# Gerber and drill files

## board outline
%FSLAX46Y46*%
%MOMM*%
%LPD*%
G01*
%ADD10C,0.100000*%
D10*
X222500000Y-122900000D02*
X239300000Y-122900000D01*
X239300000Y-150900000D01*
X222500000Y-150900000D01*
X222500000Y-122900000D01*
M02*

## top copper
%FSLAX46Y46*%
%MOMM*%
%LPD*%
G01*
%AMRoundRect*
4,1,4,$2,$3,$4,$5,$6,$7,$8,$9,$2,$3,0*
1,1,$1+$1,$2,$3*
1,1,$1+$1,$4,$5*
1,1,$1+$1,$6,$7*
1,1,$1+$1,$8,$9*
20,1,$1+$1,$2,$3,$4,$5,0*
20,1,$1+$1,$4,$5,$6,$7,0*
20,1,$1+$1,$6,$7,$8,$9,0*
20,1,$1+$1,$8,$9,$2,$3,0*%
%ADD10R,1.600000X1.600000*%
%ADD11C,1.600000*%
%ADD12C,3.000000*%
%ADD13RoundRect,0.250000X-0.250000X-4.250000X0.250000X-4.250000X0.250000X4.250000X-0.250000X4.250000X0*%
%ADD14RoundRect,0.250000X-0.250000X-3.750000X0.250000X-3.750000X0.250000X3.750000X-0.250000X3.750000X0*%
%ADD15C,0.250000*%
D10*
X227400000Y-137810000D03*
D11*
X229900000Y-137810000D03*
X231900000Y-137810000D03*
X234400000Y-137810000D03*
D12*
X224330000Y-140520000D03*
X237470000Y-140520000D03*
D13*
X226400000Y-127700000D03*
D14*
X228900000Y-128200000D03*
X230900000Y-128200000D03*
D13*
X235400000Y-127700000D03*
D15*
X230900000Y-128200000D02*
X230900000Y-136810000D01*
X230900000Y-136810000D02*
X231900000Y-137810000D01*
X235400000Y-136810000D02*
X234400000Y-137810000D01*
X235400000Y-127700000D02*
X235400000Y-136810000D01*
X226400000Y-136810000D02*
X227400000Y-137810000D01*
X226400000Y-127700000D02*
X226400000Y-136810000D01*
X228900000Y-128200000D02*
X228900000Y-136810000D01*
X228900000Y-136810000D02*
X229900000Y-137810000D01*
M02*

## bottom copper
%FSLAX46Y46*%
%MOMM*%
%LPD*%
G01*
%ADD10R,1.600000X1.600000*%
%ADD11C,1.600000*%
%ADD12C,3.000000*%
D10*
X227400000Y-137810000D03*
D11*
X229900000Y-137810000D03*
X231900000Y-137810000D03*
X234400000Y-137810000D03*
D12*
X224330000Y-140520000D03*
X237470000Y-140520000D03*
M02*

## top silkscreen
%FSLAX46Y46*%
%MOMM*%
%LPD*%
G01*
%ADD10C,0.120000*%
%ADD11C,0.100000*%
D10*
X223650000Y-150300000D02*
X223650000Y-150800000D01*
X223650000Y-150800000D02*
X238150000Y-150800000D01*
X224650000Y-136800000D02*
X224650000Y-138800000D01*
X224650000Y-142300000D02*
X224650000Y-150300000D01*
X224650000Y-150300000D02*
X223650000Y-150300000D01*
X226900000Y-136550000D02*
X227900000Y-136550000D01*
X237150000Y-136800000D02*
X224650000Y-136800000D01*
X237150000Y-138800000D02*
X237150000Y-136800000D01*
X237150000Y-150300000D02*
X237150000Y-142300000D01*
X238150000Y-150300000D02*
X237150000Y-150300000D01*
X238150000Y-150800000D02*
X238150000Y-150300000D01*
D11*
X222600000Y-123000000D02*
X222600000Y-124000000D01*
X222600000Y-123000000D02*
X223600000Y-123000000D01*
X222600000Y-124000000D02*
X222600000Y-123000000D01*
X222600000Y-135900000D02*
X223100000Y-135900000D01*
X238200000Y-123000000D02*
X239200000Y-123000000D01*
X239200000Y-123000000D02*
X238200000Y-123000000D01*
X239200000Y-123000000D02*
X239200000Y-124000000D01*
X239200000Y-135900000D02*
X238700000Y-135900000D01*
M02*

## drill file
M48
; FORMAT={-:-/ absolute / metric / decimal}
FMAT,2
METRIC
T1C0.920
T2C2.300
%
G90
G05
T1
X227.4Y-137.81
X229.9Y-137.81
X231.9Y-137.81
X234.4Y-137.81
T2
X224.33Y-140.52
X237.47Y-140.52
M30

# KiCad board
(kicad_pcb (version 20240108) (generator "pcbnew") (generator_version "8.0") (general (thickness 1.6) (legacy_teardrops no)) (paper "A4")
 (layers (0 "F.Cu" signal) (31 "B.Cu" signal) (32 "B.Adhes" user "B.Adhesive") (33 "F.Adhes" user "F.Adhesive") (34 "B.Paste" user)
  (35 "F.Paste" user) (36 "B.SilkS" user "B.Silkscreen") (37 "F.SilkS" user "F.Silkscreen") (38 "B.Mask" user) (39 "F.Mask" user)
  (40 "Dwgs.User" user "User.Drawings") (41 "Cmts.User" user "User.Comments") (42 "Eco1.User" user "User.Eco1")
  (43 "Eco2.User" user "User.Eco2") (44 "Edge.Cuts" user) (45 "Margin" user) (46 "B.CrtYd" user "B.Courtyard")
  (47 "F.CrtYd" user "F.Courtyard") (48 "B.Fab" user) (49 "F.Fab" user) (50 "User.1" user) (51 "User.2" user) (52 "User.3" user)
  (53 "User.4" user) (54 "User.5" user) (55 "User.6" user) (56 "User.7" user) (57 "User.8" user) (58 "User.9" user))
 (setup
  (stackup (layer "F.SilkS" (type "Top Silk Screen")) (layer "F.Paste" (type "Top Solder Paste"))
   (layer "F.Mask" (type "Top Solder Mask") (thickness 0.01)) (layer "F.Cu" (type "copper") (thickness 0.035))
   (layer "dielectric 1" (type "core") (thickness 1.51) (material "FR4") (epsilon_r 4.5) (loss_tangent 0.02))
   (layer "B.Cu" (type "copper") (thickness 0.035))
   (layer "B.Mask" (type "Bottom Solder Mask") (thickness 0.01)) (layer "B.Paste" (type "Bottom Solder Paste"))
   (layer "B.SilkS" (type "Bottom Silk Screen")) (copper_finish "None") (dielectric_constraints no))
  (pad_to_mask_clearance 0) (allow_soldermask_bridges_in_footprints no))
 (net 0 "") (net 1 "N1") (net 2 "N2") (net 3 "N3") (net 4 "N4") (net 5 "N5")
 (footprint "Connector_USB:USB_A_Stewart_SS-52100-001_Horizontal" (layer "F.Cu") (at 227.4 137.81)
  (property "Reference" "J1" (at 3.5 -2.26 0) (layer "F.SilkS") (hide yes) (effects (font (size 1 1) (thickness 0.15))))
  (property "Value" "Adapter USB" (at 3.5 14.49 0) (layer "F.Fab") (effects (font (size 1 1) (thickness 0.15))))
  (fp_line (start -3.75 12.49) (end -3.75 12.99) (stroke (width 0.12) (type solid)) (layer "F.SilkS"))
  (fp_line (start -3.75 12.99) (end 10.75 12.99) (stroke (width 0.12) (type solid)) (layer "F.SilkS"))
  (fp_line (start -2.75 -1.01) (end -2.75 0.99) (stroke (width 0.12) (type solid)) (layer "F.SilkS"))
  (fp_line (start -2.75 4.49) (end -2.75 12.49) (stroke (width 0.12) (type solid)) (layer "F.SilkS"))
  (fp_line (start -2.75 12.49) (end -3.75 12.49) (stroke (width 0.12) (type solid)) (layer "F.SilkS"))
  (fp_line (start -0.5 -1.26) (end 0.5 -1.26) (stroke (width 0.12) (type solid)) (layer "F.SilkS"))
  (fp_line (start 9.75 -1.01) (end -2.75 -1.01) (stroke (width 0.12) (type solid)) (layer "F.SilkS"))
  (fp_line (start 9.75 0.99) (end 9.75 -1.01) (stroke (width 0.12) (type solid)) (layer "F.SilkS"))
  (fp_line (start 9.75 12.49) (end 9.75 4.49) (stroke (width 0.12) (type solid)) (layer "F.SilkS"))
  (fp_line (start 10.75 12.49) (end 9.75 12.49) (stroke (width 0.12) (type solid)) (layer "F.SilkS"))
  (fp_line (start 10.75 12.99) (end 10.75 12.49) (stroke (width 0.12) (type solid)) (layer "F.SilkS"))
  (pad "1" thru_hole rect (at 0 0) (size 1.6 1.6) (drill 0.92) (layers "*.Cu" "*.Mask") (remove_unused_layers no) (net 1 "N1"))
  (pad "2" thru_hole circle (at 2.5 0) (size 1.6 1.6) (drill 0.92) (layers "*.Cu" "*.Mask") (remove_unused_layers no) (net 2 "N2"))
  (pad "3" thru_hole circle (at 4.5 0) (size 1.6 1.6) (drill 0.92) (layers "*.Cu" "*.Mask") (remove_unused_layers no) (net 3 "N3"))
  (pad "4" thru_hole circle (at 7 0) (size 1.6 1.6) (drill 0.92) (layers "*.Cu" "*.Mask") (remove_unused_layers no) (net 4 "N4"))
  (pad "5" thru_hole circle (at -3.07 2.71) (size 3 3) (drill 2.3) (layers "*.Cu" "*.Mask") (remove_unused_layers no) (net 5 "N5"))
  (pad "5" thru_hole circle (at 10.07 2.71) (size 3 3) (drill 2.3) (layers "*.Cu" "*.Mask") (remove_unused_layers no) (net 5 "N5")))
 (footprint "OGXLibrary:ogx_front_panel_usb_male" (layer "F.Cu") (at 222.4 122.9)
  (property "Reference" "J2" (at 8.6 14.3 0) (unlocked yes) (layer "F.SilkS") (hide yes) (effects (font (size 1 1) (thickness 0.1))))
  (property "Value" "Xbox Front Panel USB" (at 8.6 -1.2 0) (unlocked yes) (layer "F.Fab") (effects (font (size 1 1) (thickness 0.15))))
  (fp_line (start 0.2 0.1) (end 0.2 1.1) (stroke (width 0.1) (type default)) (layer "F.SilkS"))
  (fp_line (start 0.2 0.1) (end 1.2 0.1) (stroke (width 0.1) (type default)) (layer "F.SilkS"))
  (fp_line (start 0.2 1.1) (end 0.2 0.1) (stroke (width 0.1) (type default)) (layer "F.SilkS"))
  (fp_line (start 0.2 13) (end 0.7 13) (stroke (width 0.1) (type default)) (layer "F.SilkS"))
  (fp_line (start 15.8 0.1) (end 16.8 0.1) (stroke (width 0.1) (type default)) (layer "F.SilkS"))
  (fp_line (start 16.8 0.1) (end 15.8 0.1) (stroke (width 0.1) (type default)) (layer "F.SilkS"))
  (fp_line (start 16.8 0.1) (end 16.8 1.1) (stroke (width 0.1) (type default)) (layer "F.SilkS"))
  (fp_line (start 16.8 13) (end 16.3 13) (stroke (width 0.1) (type default)) (layer "F.SilkS"))
  (pad "1" smd roundrect (at 4 4.8) (size 1 9) (layers "F.Cu" "F.Paste" "F.Mask") (roundrect_rratio 0.25) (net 1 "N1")
   (thermal_bridge_angle 45))
  (pad "2" smd roundrect (at 6.5 5.3) (size 1 8) (layers "F.Cu" "F.Paste" "F.Mask") (roundrect_rratio 0.25) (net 2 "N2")
   (thermal_bridge_angle 45))
  (pad "3" smd roundrect (at 8.5 5.3) (size 1 8) (layers "F.Cu" "F.Paste" "F.Mask") (roundrect_rratio 0.25) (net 3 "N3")
   (thermal_bridge_angle 45))
  (pad "4" smd roundrect (at 13 4.8) (size 1 9) (layers "F.Cu" "F.Paste" "F.Mask") (roundrect_rratio 0.25) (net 4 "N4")
   (thermal_bridge_angle 45)))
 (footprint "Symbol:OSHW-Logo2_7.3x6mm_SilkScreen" (layer "B.Cu") (at 230.9 142.4 180)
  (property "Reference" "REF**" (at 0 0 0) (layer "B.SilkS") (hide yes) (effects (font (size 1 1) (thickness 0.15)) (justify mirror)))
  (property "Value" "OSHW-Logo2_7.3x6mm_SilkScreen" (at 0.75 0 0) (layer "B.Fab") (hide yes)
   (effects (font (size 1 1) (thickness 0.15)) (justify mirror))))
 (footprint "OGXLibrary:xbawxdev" (layer "B.Cu") (at 231.3 127.3 180)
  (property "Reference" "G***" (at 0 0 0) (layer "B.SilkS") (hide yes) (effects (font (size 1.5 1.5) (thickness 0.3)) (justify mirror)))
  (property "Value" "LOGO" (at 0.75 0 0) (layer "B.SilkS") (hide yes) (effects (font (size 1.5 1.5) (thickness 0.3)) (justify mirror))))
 (gr_rect (start 222.5 122.9) (end 239.3 150.9) (stroke (width 0.1) (type default)) (fill none) (layer "Edge.Cuts"))
 (segment (start 230.9 128.2) (end 230.9 136.81) (width 0.25) (layer "F.Cu") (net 3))
 (segment (start 230.9 136.81) (end 231.9 137.81) (width 0.25) (layer "F.Cu") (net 3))
 (segment (start 235.4 136.81) (end 234.4 137.81) (width 0.25) (layer "F.Cu") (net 4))
 (segment (start 235.4 127.7) (end 235.4 136.81) (width 0.25) (layer "F.Cu") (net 4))
 (segment (start 226.4 136.81) (end 227.4 137.81) (width 0.25) (layer "F.Cu") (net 1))
 (segment (start 226.4 127.7) (end 226.4 136.81) (width 0.25) (layer "F.Cu") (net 1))
 (segment (start 228.9 128.2) (end 228.9 136.81) (width 0.25) (layer "F.Cu") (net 2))
 (segment (start 228.9 136.81) (end 229.9 137.81) (width 0.25) (layer "F.Cu") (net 2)))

